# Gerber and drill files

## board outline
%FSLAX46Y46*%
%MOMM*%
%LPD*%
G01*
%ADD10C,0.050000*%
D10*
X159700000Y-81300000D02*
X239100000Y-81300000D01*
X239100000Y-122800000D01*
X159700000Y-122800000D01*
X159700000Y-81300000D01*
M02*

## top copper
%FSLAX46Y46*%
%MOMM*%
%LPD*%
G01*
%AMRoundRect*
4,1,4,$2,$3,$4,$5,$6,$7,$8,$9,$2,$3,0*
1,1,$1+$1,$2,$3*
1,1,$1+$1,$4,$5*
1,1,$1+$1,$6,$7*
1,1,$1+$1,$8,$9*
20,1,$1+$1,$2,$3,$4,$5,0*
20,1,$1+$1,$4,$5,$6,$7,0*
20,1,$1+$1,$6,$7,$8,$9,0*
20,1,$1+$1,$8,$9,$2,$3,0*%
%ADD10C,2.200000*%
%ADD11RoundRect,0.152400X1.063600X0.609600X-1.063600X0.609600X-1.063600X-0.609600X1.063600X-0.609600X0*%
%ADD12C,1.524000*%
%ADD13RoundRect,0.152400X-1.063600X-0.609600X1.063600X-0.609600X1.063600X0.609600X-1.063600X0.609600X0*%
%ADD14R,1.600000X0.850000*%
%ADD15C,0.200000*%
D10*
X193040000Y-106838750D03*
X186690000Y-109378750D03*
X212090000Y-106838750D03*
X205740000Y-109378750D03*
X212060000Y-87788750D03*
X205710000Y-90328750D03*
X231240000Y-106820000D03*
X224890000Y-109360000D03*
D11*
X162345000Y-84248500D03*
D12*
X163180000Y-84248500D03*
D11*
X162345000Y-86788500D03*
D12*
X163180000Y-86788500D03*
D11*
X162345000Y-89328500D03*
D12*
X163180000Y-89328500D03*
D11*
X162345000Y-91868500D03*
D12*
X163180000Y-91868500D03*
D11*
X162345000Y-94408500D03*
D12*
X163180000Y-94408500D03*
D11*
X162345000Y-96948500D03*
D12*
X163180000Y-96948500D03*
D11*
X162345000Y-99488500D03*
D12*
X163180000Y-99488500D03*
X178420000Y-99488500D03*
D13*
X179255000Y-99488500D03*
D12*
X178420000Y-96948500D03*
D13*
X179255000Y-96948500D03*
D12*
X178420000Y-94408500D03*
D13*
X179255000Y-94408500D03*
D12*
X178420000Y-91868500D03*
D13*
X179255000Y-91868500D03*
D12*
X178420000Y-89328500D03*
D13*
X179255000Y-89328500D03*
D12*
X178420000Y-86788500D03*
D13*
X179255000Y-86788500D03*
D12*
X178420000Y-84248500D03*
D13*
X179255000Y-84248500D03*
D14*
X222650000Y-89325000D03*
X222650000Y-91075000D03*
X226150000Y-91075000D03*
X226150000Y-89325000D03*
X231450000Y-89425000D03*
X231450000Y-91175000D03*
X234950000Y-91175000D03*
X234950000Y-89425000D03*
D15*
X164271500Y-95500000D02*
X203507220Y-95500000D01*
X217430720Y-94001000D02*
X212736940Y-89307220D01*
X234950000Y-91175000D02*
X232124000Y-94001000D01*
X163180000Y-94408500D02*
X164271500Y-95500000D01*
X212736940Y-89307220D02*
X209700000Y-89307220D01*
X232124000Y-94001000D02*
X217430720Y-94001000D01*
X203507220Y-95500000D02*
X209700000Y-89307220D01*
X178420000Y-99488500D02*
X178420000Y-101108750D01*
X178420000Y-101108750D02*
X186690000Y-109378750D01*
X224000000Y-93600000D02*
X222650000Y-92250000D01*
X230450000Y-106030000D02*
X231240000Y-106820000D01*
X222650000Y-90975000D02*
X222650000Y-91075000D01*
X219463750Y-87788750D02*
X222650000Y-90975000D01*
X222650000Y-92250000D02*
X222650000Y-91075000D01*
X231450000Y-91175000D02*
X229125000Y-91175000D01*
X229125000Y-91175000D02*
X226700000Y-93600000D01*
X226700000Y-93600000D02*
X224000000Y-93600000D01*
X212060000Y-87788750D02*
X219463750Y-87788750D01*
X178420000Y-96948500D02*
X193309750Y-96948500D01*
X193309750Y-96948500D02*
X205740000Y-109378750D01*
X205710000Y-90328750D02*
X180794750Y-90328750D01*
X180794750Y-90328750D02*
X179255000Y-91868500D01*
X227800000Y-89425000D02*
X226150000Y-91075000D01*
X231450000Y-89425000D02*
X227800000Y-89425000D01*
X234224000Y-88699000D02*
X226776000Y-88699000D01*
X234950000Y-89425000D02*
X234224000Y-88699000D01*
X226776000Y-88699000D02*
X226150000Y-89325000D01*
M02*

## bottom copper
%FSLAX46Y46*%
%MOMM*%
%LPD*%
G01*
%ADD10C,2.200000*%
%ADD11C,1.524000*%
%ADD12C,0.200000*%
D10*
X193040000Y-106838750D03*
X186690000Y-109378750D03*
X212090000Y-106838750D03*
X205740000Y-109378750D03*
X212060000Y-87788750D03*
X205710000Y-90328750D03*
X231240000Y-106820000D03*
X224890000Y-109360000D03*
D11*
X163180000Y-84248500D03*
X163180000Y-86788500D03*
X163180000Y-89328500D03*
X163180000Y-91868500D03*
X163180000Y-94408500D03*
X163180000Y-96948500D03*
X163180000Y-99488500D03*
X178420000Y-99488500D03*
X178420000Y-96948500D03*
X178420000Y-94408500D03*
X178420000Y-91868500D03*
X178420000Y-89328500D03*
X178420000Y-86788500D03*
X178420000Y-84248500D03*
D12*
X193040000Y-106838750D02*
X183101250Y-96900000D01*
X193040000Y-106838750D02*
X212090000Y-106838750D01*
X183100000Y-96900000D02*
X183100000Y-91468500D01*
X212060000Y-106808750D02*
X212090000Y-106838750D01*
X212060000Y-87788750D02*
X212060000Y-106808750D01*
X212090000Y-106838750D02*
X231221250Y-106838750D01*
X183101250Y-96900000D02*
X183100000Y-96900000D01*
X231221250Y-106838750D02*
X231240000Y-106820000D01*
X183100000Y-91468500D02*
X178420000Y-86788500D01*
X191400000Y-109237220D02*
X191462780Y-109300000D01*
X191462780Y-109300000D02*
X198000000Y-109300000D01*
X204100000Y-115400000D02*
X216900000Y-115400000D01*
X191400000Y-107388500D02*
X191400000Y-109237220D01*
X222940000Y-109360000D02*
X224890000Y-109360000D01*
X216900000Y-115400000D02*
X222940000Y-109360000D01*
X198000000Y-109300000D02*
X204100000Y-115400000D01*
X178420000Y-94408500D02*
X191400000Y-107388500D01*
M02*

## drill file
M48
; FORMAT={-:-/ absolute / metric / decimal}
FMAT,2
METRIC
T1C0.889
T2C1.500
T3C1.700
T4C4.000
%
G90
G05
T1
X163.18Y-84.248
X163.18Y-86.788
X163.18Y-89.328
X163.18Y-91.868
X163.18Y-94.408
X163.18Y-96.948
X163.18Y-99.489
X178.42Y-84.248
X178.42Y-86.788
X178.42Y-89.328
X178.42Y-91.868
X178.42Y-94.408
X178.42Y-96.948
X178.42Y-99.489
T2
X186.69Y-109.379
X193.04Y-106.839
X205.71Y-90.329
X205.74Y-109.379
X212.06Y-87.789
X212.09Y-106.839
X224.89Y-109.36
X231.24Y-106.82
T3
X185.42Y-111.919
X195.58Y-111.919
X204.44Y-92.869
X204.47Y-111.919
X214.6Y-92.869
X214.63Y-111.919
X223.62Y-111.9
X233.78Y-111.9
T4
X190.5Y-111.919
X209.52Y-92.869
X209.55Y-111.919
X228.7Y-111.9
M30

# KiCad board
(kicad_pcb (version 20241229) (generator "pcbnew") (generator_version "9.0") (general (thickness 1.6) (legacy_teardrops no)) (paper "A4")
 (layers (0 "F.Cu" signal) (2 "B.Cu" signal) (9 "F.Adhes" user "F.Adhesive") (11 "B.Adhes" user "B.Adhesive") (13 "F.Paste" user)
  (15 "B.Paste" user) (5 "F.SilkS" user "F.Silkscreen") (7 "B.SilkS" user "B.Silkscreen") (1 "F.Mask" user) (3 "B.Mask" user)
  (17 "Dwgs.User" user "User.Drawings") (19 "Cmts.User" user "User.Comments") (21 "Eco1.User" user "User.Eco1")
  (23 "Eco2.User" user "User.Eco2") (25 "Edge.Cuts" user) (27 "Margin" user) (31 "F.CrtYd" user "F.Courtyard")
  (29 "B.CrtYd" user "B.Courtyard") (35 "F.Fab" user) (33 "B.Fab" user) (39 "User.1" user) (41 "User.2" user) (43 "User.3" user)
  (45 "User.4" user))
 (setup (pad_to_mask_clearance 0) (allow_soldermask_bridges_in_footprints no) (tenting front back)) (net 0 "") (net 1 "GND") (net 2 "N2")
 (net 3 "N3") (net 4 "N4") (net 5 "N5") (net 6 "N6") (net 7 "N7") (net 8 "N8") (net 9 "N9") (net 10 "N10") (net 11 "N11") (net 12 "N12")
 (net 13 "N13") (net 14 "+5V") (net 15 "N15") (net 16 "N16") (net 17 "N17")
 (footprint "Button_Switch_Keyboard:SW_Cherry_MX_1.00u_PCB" (layer "F.Cu") (at 193.04 106.83875)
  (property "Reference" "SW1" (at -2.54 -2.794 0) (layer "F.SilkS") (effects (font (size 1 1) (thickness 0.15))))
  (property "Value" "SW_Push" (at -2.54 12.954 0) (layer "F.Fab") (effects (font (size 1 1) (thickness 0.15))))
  (pad "" np_thru_hole circle (at -7.62 5.08) (size 1.7 1.7) (drill 1.7) (layers "*.Cu" "*.Mask"))
  (pad "" np_thru_hole circle (at -2.54 5.08) (size 4 4) (drill 4) (layers "*.Cu" "*.Mask"))
  (pad "" np_thru_hole circle (at 2.54 5.08) (size 1.7 1.7) (drill 1.7) (layers "*.Cu" "*.Mask"))
  (pad "1" thru_hole circle (at 0 0) (size 2.2 2.2) (drill 1.5) (layers "*.Cu" "*.Mask") (remove_unused_layers no) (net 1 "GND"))
  (pad "2" thru_hole circle (at -6.35 2.54) (size 2.2 2.2) (drill 1.5) (layers "*.Cu" "*.Mask") (remove_unused_layers no) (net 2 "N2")))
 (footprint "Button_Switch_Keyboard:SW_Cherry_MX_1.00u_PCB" (layer "F.Cu") (at 212.09 106.83875)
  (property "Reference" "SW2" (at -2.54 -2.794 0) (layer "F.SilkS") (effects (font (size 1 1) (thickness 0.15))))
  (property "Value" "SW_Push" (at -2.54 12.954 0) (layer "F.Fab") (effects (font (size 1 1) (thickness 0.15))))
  (pad "" np_thru_hole circle (at -7.62 5.08) (size 1.7 1.7) (drill 1.7) (layers "*.Cu" "*.Mask"))
  (pad "" np_thru_hole circle (at -2.54 5.08) (size 4 4) (drill 4) (layers "*.Cu" "*.Mask"))
  (pad "" np_thru_hole circle (at 2.54 5.08) (size 1.7 1.7) (drill 1.7) (layers "*.Cu" "*.Mask"))
  (pad "1" thru_hole circle (at 0 0) (size 2.2 2.2) (drill 1.5) (layers "*.Cu" "*.Mask") (remove_unused_layers no) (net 1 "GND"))
  (pad "2" thru_hole circle (at -6.35 2.54) (size 2.2 2.2) (drill 1.5) (layers "*.Cu" "*.Mask") (remove_unused_layers no) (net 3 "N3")))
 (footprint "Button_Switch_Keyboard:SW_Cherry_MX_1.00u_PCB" (layer "F.Cu") (at 212.06 87.78875)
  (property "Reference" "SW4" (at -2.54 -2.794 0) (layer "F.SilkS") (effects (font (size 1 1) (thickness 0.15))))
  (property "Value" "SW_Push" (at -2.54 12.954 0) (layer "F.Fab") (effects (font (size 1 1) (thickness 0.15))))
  (pad "" np_thru_hole circle (at -7.62 5.08) (size 1.7 1.7) (drill 1.7) (layers "*.Cu" "*.Mask"))
  (pad "" np_thru_hole circle (at -2.54 5.08) (size 4 4) (drill 4) (layers "*.Cu" "*.Mask"))
  (pad "" np_thru_hole circle (at 2.54 5.08) (size 1.7 1.7) (drill 1.7) (layers "*.Cu" "*.Mask"))
  (pad "1" thru_hole circle (at 0 0) (size 2.2 2.2) (drill 1.5) (layers "*.Cu" "*.Mask") (remove_unused_layers no) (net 1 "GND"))
  (pad "2" thru_hole circle (at -6.35 2.54) (size 2.2 2.2) (drill 1.5) (layers "*.Cu" "*.Mask") (remove_unused_layers no) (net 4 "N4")))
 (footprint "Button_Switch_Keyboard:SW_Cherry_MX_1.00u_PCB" (layer "F.Cu") (at 231.24 106.82)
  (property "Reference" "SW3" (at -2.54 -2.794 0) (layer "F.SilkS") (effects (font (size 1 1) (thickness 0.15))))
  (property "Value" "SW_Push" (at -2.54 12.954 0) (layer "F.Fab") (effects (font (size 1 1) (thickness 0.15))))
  (pad "" np_thru_hole circle (at -7.62 5.08) (size 1.7 1.7) (drill 1.7) (layers "*.Cu" "*.Mask"))
  (pad "" np_thru_hole circle (at -2.54 5.08) (size 4 4) (drill 4) (layers "*.Cu" "*.Mask"))
  (pad "" np_thru_hole circle (at 2.54 5.08) (size 1.7 1.7) (drill 1.7) (layers "*.Cu" "*.Mask"))
  (pad "1" thru_hole circle (at 0 0) (size 2.2 2.2) (drill 1.5) (layers "*.Cu" "*.Mask") (remove_unused_layers no) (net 1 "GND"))
  (pad "2" thru_hole circle (at -6.35 2.54) (size 2.2 2.2) (drill 1.5) (layers "*.Cu" "*.Mask") (remove_unused_layers no) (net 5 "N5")))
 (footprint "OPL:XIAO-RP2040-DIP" (layer "F.Cu") (at 170.8 91.8685)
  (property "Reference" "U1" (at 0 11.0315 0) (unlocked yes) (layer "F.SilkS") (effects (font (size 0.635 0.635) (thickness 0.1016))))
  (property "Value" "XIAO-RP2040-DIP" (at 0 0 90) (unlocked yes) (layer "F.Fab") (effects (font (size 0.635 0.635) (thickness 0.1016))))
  (pad "1" smd roundrect (at -8.455 -7.62 180) (size 2.432 1.524) (layers "F.Cu" "F.Mask") (roundrect_rratio 0.1) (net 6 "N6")
   (thermal_bridge_angle 45))
  (pad "1" thru_hole circle (at -7.62 -7.62 180) (size 1.524 1.524) (drill 0.889) (layers "*.Cu" "*.Mask") (remove_unused_layers no)
   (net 6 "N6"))
  (pad "2" smd roundrect (at -8.455 -5.08 180) (size 2.432 1.524) (layers "F.Cu" "F.Mask") (roundrect_rratio 0.1) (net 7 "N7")
   (thermal_bridge_angle 45))
  (pad "2" thru_hole circle (at -7.62 -5.08 180) (size 1.524 1.524) (drill 0.889) (layers "*.Cu" "*.Mask") (remove_unused_layers no)
   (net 7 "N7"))
  (pad "3" smd roundrect (at -8.455 -2.54 180) (size 2.432 1.524) (layers "F.Cu" "F.Mask") (roundrect_rratio 0.1) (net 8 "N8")
   (thermal_bridge_angle 45))
  (pad "3" thru_hole circle (at -7.62 -2.54 180) (size 1.524 1.524) (drill 0.889) (layers "*.Cu" "*.Mask") (remove_unused_layers no)
   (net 8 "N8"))
  (pad "4" smd roundrect (at -8.455 0 180) (size 2.432 1.524) (layers "F.Cu" "F.Mask") (roundrect_rratio 0.1) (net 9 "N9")
   (thermal_bridge_angle 45))
  (pad "4" thru_hole circle (at -7.62 0 180) (size 1.524 1.524) (drill 0.889) (layers "*.Cu" "*.Mask") (remove_unused_layers no)
   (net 9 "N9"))
  (pad "5" smd roundrect (at -8.455 2.54 180) (size 2.432 1.524) (layers "F.Cu" "F.Mask") (roundrect_rratio 0.1) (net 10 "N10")
   (thermal_bridge_angle 45))
  (pad "5" thru_hole circle (at -7.62 2.54 180) (size 1.524 1.524) (drill 0.889) (layers "*.Cu" "*.Mask") (remove_unused_layers no)
   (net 10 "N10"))
  (pad "6" smd roundrect (at -8.455 5.08 180) (size 2.432 1.524) (layers "F.Cu" "F.Mask") (roundrect_rratio 0.1) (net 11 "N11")
   (thermal_bridge_angle 45))
  (pad "6" thru_hole circle (at -7.62 5.08 180) (size 1.524 1.524) (drill 0.889) (layers "*.Cu" "*.Mask") (remove_unused_layers no)
   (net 11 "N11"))
  (pad "7" smd roundrect (at -8.455 7.62 180) (size 2.432 1.524) (layers "F.Cu" "F.Mask") (roundrect_rratio 0.1) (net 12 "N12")
   (thermal_bridge_angle 45))
  (pad "7" thru_hole circle (at -7.62 7.62 180) (size 1.524 1.524) (drill 0.889) (layers "*.Cu" "*.Mask") (remove_unused_layers no)
   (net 12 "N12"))
  (pad "8" thru_hole circle (at 7.62 7.62) (size 1.524 1.524) (drill 0.889) (layers "*.Cu" "*.Mask") (remove_unused_layers no) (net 2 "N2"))
  (pad "8" smd roundrect (at 8.455 7.62) (size 2.432 1.524) (layers "F.Cu" "F.Mask") (roundrect_rratio 0.1) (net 2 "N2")
   (thermal_bridge_angle 45))
  (pad "9" thru_hole circle (at 7.62 5.08) (size 1.524 1.524) (drill 0.889) (layers "*.Cu" "*.Mask") (remove_unused_layers no) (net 3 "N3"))
  (pad "9" smd roundrect (at 8.455 5.08) (size 2.432 1.524) (layers "F.Cu" "F.Mask") (roundrect_rratio 0.1) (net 3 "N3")
   (thermal_bridge_angle 45))
  (pad "10" thru_hole circle (at 7.62 2.54) (size 1.524 1.524) (drill 0.889) (layers "*.Cu" "*.Mask") (remove_unused_layers no) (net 5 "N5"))
  (pad "10" smd roundrect (at 8.455 2.54) (size 2.432 1.524) (layers "F.Cu" "F.Mask") (roundrect_rratio 0.1) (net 5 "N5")
   (thermal_bridge_angle 45))
  (pad "11" thru_hole circle (at 7.62 0) (size 1.524 1.524) (drill 0.889) (layers "*.Cu" "*.Mask") (remove_unused_layers no) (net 4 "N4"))
  (pad "11" smd roundrect (at 8.455 0) (size 2.432 1.524) (layers "F.Cu" "F.Mask") (roundrect_rratio 0.1) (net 4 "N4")
   (thermal_bridge_angle 45))
  (pad "12" thru_hole circle (at 7.62 -2.54) (size 1.524 1.524) (drill 0.889) (layers "*.Cu" "*.Mask") (remove_unused_layers no)
   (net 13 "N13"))
  (pad "12" smd roundrect (at 8.455 -2.54) (size 2.432 1.524) (layers "F.Cu" "F.Mask") (roundrect_rratio 0.1) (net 13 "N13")
   (thermal_bridge_angle 45))
  (pad "13" thru_hole circle (at 7.62 -5.08) (size 1.524 1.524) (drill 0.889) (layers "*.Cu" "*.Mask") (remove_unused_layers no)
   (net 1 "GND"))
  (pad "13" smd roundrect (at 8.455 -5.08) (size 2.432 1.524) (layers "F.Cu" "F.Mask") (roundrect_rratio 0.1) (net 1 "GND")
   (thermal_bridge_angle 45))
  (pad "14" thru_hole circle (at 7.62 -7.62) (size 1.524 1.524) (drill 0.889) (layers "*.Cu" "*.Mask") (remove_unused_layers no)
   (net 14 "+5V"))
  (pad "14" smd roundrect (at 8.455 -7.62) (size 2.432 1.524) (layers "F.Cu" "F.Mask") (roundrect_rratio 0.1) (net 14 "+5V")
   (thermal_bridge_angle 45)))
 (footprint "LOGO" (layer "F.Cu") (at 190.1 92.7)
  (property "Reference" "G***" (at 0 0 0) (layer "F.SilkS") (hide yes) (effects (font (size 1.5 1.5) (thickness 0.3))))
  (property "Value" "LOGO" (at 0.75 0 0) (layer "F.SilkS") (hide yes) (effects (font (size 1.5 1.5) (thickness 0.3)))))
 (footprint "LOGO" (layer "F.Cu") (at 170.1 110.6)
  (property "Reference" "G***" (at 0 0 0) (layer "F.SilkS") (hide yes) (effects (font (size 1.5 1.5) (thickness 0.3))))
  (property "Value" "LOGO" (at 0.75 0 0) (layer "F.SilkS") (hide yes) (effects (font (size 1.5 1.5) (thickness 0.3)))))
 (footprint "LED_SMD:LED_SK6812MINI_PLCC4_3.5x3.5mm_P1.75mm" (layer "F.Cu") (at 224.4 90.2)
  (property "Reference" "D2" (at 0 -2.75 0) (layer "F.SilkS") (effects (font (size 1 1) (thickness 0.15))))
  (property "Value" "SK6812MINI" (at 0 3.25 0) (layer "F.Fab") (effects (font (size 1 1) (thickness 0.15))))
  (pad "1" smd rect (at -1.75 -0.875) (size 1.6 0.85) (layers "F.Cu" "F.Mask" "F.Paste") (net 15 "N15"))
  (pad "2" smd rect (at -1.75 0.875) (size 1.6 0.85) (layers "F.Cu" "F.Mask" "F.Paste") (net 1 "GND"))
  (pad "3" smd rect (at 1.75 0.875) (size 1.6 0.85) (layers "F.Cu" "F.Mask" "F.Paste") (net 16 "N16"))
  (pad "4" smd rect (at 1.75 -0.875) (size 1.6 0.85) (layers "F.Cu" "F.Mask" "F.Paste") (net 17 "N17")))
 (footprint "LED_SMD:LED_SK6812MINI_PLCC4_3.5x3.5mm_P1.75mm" (layer "F.Cu") (at 233.2 90.3)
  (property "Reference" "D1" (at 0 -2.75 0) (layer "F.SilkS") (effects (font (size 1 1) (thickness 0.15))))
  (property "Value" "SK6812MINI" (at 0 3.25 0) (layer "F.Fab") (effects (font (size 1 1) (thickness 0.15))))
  (pad "1" smd rect (at -1.75 -0.875) (size 1.6 0.85) (layers "F.Cu" "F.Mask" "F.Paste") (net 16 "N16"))
  (pad "2" smd rect (at -1.75 0.875) (size 1.6 0.85) (layers "F.Cu" "F.Mask" "F.Paste") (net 1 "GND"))
  (pad "3" smd rect (at 1.75 0.875) (size 1.6 0.85) (layers "F.Cu" "F.Mask" "F.Paste") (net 10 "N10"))
  (pad "4" smd rect (at 1.75 -0.875) (size 1.6 0.85) (layers "F.Cu" "F.Mask" "F.Paste") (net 17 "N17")))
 (gr_rect (start 159.7 81.3) (end 239.1 122.8) (stroke (width 0.05) (type default)) (fill no) (layer "Edge.Cuts"))
 (segment (start 164.2715 95.5) (end 203.50722 95.5) (width 0.2) (layer "F.Cu") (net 10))
 (segment (start 217.43072 94.001) (end 212.73694 89.30722) (width 0.2) (layer "F.Cu") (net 10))
 (segment (start 234.95 91.175) (end 232.124 94.001) (width 0.2) (layer "F.Cu") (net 10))
 (segment (start 163.18 94.4085) (end 164.2715 95.5) (width 0.2) (layer "F.Cu") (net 10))
 (segment (start 212.73694 89.30722) (end 209.7 89.30722) (width 0.2) (layer "F.Cu") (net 10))
 (segment (start 232.124 94.001) (end 217.43072 94.001) (width 0.2) (layer "F.Cu") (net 10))
 (segment (start 203.50722 95.5) (end 209.7 89.30722) (width 0.2) (layer "F.Cu") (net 10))
 (segment (start 178.42 99.4885) (end 178.42 101.10875) (width 0.2) (layer "F.Cu") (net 2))
 (segment (start 178.42 101.10875) (end 186.69 109.37875) (width 0.2) (layer "F.Cu") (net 2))
 (segment (start 224 93.6) (end 222.65 92.25) (width 0.2) (layer "F.Cu") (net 1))
 (segment (start 230.45 106.03) (end 231.24 106.82) (width 0.2) (layer "F.Cu") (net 1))
 (segment (start 222.65 90.975) (end 222.65 91.075) (width 0.2) (layer "F.Cu") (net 1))
 (segment (start 219.46375 87.78875) (end 222.65 90.975) (width 0.2) (layer "F.Cu") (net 1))
 (segment (start 222.65 92.25) (end 222.65 91.075) (width 0.2) (layer "F.Cu") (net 1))
 (segment (start 231.45 91.175) (end 229.125 91.175) (width 0.2) (layer "F.Cu") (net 1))
 (segment (start 229.125 91.175) (end 226.7 93.6) (width 0.2) (layer "F.Cu") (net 1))
 (segment (start 226.7 93.6) (end 224 93.6) (width 0.2) (layer "F.Cu") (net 1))
 (segment (start 212.06 87.78875) (end 219.46375 87.78875) (width 0.2) (layer "F.Cu") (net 1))
 (segment (start 193.04 106.83875) (end 183.10125 96.9) (width 0.2) (layer "B.Cu") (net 1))
 (segment (start 193.04 106.83875) (end 212.09 106.83875) (width 0.2) (layer "B.Cu") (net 1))
 (segment (start 183.1 96.9) (end 183.1 91.4685) (width 0.2) (layer "B.Cu") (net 1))
 (segment (start 212.06 106.80875) (end 212.09 106.83875) (width 0.2) (layer "B.Cu") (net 1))
 (segment (start 212.06 87.78875) (end 212.06 106.80875) (width 0.2) (layer "B.Cu") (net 1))
 (segment (start 212.09 106.83875) (end 231.22125 106.83875) (width 0.2) (layer "B.Cu") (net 1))
 (segment (start 183.10125 96.9) (end 183.1 96.9) (width 0.2) (layer "B.Cu") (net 1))
 (segment (start 231.22125 106.83875) (end 231.24 106.82) (width 0.2) (layer "B.Cu") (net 1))
 (segment (start 183.1 91.4685) (end 178.42 86.7885) (width 0.2) (layer "B.Cu") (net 1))
 (segment (start 178.42 96.9485) (end 193.30975 96.9485) (width 0.2) (layer "F.Cu") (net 3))
 (segment (start 193.30975 96.9485) (end 205.74 109.37875) (width 0.2) (layer "F.Cu") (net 3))
 (segment (start 191.4 109.23722) (end 191.46278 109.3) (width 0.2) (layer "B.Cu") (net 5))
 (segment (start 191.46278 109.3) (end 198 109.3) (width 0.2) (layer "B.Cu") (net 5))
 (segment (start 204.1 115.4) (end 216.9 115.4) (width 0.2) (layer "B.Cu") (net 5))
 (segment (start 191.4 107.3885) (end 191.4 109.23722) (width 0.2) (layer "B.Cu") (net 5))
 (segment (start 222.94 109.36) (end 224.89 109.36) (width 0.2) (layer "B.Cu") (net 5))
 (segment (start 216.9 115.4) (end 222.94 109.36) (width 0.2) (layer "B.Cu") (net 5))
 (segment (start 198 109.3) (end 204.1 115.4) (width 0.2) (layer "B.Cu") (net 5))
 (segment (start 178.42 94.4085) (end 191.4 107.3885) (width 0.2) (layer "B.Cu") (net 5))
 (segment (start 205.71 90.32875) (end 180.79475 90.32875) (width 0.2) (layer "F.Cu") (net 4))
 (segment (start 180.79475 90.32875) (end 179.255 91.8685) (width 0.2) (layer "F.Cu") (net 4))
 (segment (start 227.8 89.425) (end 226.15 91.075) (width 0.2) (layer "F.Cu") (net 16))
 (segment (start 231.45 89.425) (end 227.8 89.425) (width 0.2) (layer "F.Cu") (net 16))
 (segment (start 234.224 88.699) (end 226.776 88.699) (width 0.2) (layer "F.Cu") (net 17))
 (segment (start 234.95 89.425) (end 234.224 88.699) (width 0.2) (layer "F.Cu") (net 17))
 (segment (start 226.776 88.699) (end 226.15 89.325) (width 0.2) (layer "F.Cu") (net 17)))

